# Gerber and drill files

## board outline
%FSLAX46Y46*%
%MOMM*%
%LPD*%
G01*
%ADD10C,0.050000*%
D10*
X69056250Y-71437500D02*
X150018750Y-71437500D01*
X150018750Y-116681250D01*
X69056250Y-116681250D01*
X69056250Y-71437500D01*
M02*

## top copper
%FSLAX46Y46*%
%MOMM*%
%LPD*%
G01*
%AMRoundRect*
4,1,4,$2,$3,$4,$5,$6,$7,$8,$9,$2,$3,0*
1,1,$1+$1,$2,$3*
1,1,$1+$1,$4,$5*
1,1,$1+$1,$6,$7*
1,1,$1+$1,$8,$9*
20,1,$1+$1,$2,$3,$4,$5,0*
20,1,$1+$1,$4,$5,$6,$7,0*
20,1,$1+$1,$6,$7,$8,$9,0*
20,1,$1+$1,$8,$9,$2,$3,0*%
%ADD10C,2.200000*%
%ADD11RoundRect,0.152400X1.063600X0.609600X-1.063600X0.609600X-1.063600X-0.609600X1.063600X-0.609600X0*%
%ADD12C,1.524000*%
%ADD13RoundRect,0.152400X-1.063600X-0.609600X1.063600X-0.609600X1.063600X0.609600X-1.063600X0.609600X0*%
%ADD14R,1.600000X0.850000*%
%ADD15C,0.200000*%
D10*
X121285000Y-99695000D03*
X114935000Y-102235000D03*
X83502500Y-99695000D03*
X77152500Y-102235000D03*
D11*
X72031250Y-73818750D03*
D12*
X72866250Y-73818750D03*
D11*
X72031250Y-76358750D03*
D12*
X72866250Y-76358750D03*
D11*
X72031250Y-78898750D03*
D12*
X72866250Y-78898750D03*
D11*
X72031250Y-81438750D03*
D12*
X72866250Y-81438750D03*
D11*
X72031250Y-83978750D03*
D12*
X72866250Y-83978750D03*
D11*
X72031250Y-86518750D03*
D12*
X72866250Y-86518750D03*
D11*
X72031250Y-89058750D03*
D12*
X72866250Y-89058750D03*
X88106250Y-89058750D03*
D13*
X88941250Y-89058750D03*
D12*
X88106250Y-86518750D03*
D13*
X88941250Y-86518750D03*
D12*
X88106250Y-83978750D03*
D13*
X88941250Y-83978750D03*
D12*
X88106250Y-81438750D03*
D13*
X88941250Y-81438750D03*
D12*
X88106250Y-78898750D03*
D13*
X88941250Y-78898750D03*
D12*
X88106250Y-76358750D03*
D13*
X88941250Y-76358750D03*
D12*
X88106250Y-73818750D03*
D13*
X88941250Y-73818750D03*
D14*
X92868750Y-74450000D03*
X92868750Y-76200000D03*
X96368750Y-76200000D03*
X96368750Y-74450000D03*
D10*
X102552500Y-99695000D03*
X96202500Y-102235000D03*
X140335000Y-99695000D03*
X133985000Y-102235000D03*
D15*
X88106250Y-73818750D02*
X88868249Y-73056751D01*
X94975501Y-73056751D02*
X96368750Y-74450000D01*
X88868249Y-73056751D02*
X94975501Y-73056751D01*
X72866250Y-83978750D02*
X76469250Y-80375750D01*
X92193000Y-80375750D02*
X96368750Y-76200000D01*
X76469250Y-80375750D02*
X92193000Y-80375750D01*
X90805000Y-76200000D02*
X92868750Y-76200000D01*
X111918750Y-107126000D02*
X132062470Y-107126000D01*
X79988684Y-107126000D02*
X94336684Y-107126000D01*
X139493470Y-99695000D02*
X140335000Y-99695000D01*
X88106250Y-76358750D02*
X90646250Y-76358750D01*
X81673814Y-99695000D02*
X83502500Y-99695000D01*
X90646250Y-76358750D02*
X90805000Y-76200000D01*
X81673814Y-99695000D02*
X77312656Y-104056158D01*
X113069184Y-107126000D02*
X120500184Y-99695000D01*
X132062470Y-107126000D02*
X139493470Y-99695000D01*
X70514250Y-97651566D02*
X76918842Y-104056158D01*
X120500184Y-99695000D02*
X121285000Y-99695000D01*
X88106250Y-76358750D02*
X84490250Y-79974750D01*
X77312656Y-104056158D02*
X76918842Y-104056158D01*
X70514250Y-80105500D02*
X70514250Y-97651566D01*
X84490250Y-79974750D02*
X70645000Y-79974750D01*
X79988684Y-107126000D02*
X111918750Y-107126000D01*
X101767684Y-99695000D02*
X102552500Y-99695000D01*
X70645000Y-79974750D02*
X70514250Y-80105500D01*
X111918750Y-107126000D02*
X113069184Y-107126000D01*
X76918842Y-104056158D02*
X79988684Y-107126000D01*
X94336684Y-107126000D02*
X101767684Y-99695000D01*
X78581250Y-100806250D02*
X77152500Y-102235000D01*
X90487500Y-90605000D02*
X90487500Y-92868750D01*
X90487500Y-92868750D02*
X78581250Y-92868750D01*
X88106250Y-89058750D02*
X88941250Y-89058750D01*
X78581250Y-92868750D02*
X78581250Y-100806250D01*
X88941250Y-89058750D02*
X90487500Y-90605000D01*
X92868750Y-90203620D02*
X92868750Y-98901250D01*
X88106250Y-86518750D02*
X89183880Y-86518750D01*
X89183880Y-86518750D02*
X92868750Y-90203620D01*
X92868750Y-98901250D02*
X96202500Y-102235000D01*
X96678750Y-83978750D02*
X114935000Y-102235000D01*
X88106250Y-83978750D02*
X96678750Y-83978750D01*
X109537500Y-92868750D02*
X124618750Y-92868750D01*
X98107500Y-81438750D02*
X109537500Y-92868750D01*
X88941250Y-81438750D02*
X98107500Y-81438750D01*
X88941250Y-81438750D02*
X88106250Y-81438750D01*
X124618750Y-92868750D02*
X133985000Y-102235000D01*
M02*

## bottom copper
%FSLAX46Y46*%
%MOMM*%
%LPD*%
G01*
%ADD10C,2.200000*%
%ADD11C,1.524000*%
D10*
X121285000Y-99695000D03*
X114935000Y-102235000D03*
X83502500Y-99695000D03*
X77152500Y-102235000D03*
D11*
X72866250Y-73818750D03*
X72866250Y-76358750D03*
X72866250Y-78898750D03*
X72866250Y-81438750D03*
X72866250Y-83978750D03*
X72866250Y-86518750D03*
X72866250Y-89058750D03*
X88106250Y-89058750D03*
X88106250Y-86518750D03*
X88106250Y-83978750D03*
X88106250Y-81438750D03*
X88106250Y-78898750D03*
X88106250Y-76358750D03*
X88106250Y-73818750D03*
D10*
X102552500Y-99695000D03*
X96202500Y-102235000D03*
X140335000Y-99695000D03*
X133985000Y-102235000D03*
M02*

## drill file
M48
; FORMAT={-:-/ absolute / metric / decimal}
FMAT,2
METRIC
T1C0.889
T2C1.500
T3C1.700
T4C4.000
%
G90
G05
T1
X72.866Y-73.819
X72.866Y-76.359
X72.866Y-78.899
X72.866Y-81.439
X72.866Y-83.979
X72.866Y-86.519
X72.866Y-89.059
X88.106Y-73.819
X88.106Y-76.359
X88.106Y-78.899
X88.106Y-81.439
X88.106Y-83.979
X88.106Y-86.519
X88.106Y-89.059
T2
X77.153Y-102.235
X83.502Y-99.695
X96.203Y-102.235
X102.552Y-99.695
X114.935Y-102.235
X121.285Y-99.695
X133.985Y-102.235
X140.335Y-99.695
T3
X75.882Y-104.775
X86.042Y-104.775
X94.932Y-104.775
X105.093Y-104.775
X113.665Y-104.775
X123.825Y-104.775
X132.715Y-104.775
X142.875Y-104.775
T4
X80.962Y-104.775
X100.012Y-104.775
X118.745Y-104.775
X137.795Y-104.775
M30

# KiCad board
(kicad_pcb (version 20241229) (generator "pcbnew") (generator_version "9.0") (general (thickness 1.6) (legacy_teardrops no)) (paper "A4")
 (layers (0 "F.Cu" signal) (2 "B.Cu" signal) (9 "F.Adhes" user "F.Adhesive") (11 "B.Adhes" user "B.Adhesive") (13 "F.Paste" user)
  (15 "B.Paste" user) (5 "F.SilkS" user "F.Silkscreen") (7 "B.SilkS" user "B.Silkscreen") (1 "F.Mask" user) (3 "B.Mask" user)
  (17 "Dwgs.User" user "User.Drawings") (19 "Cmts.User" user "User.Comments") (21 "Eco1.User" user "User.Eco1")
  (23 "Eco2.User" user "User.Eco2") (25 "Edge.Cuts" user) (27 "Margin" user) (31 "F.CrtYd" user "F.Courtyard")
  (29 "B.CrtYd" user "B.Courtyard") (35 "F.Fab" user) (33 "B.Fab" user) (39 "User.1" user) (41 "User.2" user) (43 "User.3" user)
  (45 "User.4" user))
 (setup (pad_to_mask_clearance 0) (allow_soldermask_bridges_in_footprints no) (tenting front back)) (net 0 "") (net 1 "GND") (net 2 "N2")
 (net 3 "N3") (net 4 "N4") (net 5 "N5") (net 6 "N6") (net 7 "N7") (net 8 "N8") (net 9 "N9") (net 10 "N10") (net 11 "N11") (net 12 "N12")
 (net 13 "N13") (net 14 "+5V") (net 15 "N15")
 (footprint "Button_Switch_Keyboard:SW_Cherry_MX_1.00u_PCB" (layer "F.Cu") (at 121.285 99.695)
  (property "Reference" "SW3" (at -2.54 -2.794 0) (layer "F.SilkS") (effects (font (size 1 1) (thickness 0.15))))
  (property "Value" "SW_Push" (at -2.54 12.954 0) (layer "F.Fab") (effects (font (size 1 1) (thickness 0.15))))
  (pad "" np_thru_hole circle (at -7.62 5.08) (size 1.7 1.7) (drill 1.7) (layers "*.Cu" "*.Mask"))
  (pad "" np_thru_hole circle (at -2.54 5.08) (size 4 4) (drill 4) (layers "*.Cu" "*.Mask"))
  (pad "" np_thru_hole circle (at 2.54 5.08) (size 1.7 1.7) (drill 1.7) (layers "*.Cu" "*.Mask"))
  (pad "1" thru_hole circle (at 0 0) (size 2.2 2.2) (drill 1.5) (layers "*.Cu" "*.Mask") (remove_unused_layers no) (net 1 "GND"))
  (pad "2" thru_hole circle (at -6.35 2.54) (size 2.2 2.2) (drill 1.5) (layers "*.Cu" "*.Mask") (remove_unused_layers no) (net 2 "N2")))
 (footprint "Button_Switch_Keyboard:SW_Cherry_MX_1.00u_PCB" (layer "F.Cu") (at 83.5025 99.695)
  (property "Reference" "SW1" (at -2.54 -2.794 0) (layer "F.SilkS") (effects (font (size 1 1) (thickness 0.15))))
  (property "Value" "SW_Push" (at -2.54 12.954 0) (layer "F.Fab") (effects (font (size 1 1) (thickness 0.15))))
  (pad "" np_thru_hole circle (at -7.62 5.08) (size 1.7 1.7) (drill 1.7) (layers "*.Cu" "*.Mask"))
  (pad "" np_thru_hole circle (at -2.54 5.08) (size 4 4) (drill 4) (layers "*.Cu" "*.Mask"))
  (pad "" np_thru_hole circle (at 2.54 5.08) (size 1.7 1.7) (drill 1.7) (layers "*.Cu" "*.Mask"))
  (pad "1" thru_hole circle (at 0 0) (size 2.2 2.2) (drill 1.5) (layers "*.Cu" "*.Mask") (remove_unused_layers no) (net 1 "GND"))
  (pad "2" thru_hole circle (at -6.35 2.54) (size 2.2 2.2) (drill 1.5) (layers "*.Cu" "*.Mask") (remove_unused_layers no) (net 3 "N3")))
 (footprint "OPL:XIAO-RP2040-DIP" (layer "F.Cu") (at 80.48625 81.43875)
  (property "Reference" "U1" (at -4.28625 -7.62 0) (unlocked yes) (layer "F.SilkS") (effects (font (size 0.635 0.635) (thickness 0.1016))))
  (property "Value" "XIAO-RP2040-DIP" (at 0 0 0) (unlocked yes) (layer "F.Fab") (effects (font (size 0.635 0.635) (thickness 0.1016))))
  (pad "1" smd roundrect (at -8.455 -7.62 180) (size 2.432 1.524) (layers "F.Cu" "F.Mask") (roundrect_rratio 0.1) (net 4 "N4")
   (thermal_bridge_angle 45))
  (pad "1" thru_hole circle (at -7.62 -7.62 180) (size 1.524 1.524) (drill 0.889) (layers "*.Cu" "*.Mask") (remove_unused_layers no)
   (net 4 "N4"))
  (pad "2" smd roundrect (at -8.455 -5.08 180) (size 2.432 1.524) (layers "F.Cu" "F.Mask") (roundrect_rratio 0.1) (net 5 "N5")
   (thermal_bridge_angle 45))
  (pad "2" thru_hole circle (at -7.62 -5.08 180) (size 1.524 1.524) (drill 0.889) (layers "*.Cu" "*.Mask") (remove_unused_layers no)
   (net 5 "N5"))
  (pad "3" smd roundrect (at -8.455 -2.54 180) (size 2.432 1.524) (layers "F.Cu" "F.Mask") (roundrect_rratio 0.1) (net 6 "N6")
   (thermal_bridge_angle 45))
  (pad "3" thru_hole circle (at -7.62 -2.54 180) (size 1.524 1.524) (drill 0.889) (layers "*.Cu" "*.Mask") (remove_unused_layers no)
   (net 6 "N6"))
  (pad "4" smd roundrect (at -8.455 0 180) (size 2.432 1.524) (layers "F.Cu" "F.Mask") (roundrect_rratio 0.1) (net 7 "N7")
   (thermal_bridge_angle 45))
  (pad "4" thru_hole circle (at -7.62 0 180) (size 1.524 1.524) (drill 0.889) (layers "*.Cu" "*.Mask") (remove_unused_layers no)
   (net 7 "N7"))
  (pad "5" smd roundrect (at -8.455 2.54 180) (size 2.432 1.524) (layers "F.Cu" "F.Mask") (roundrect_rratio 0.1) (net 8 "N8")
   (thermal_bridge_angle 45))
  (pad "5" thru_hole circle (at -7.62 2.54 180) (size 1.524 1.524) (drill 0.889) (layers "*.Cu" "*.Mask") (remove_unused_layers no)
   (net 8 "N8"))
  (pad "6" smd roundrect (at -8.455 5.08 180) (size 2.432 1.524) (layers "F.Cu" "F.Mask") (roundrect_rratio 0.1) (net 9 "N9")
   (thermal_bridge_angle 45))
  (pad "6" thru_hole circle (at -7.62 5.08 180) (size 1.524 1.524) (drill 0.889) (layers "*.Cu" "*.Mask") (remove_unused_layers no)
   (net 9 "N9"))
  (pad "7" smd roundrect (at -8.455 7.62 180) (size 2.432 1.524) (layers "F.Cu" "F.Mask") (roundrect_rratio 0.1) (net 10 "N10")
   (thermal_bridge_angle 45))
  (pad "7" thru_hole circle (at -7.62 7.62 180) (size 1.524 1.524) (drill 0.889) (layers "*.Cu" "*.Mask") (remove_unused_layers no)
   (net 10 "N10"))
  (pad "8" thru_hole circle (at 7.62 7.62) (size 1.524 1.524) (drill 0.889) (layers "*.Cu" "*.Mask") (remove_unused_layers no) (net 3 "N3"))
  (pad "8" smd roundrect (at 8.455 7.62) (size 2.432 1.524) (layers "F.Cu" "F.Mask") (roundrect_rratio 0.1) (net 3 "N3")
   (thermal_bridge_angle 45))
  (pad "9" thru_hole circle (at 7.62 5.08) (size 1.524 1.524) (drill 0.889) (layers "*.Cu" "*.Mask") (remove_unused_layers no)
   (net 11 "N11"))
  (pad "9" smd roundrect (at 8.455 5.08) (size 2.432 1.524) (layers "F.Cu" "F.Mask") (roundrect_rratio 0.1) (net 11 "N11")
   (thermal_bridge_angle 45))
  (pad "10" thru_hole circle (at 7.62 2.54) (size 1.524 1.524) (drill 0.889) (layers "*.Cu" "*.Mask") (remove_unused_layers no) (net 2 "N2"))
  (pad "10" smd roundrect (at 8.455 2.54) (size 2.432 1.524) (layers "F.Cu" "F.Mask") (roundrect_rratio 0.1) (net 2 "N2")
   (thermal_bridge_angle 45))
  (pad "11" thru_hole circle (at 7.62 0) (size 1.524 1.524) (drill 0.889) (layers "*.Cu" "*.Mask") (remove_unused_layers no) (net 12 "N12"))
  (pad "11" smd roundrect (at 8.455 0) (size 2.432 1.524) (layers "F.Cu" "F.Mask") (roundrect_rratio 0.1) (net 12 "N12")
   (thermal_bridge_angle 45))
  (pad "12" thru_hole circle (at 7.62 -2.54) (size 1.524 1.524) (drill 0.889) (layers "*.Cu" "*.Mask") (remove_unused_layers no)
   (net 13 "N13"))
  (pad "12" smd roundrect (at 8.455 -2.54) (size 2.432 1.524) (layers "F.Cu" "F.Mask") (roundrect_rratio 0.1) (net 13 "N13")
   (thermal_bridge_angle 45))
  (pad "13" thru_hole circle (at 7.62 -5.08) (size 1.524 1.524) (drill 0.889) (layers "*.Cu" "*.Mask") (remove_unused_layers no)
   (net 1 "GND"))
  (pad "13" smd roundrect (at 8.455 -5.08) (size 2.432 1.524) (layers "F.Cu" "F.Mask") (roundrect_rratio 0.1) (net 1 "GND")
   (thermal_bridge_angle 45))
  (pad "14" thru_hole circle (at 7.62 -7.62) (size 1.524 1.524) (drill 0.889) (layers "*.Cu" "*.Mask") (remove_unused_layers no)
   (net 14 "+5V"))
  (pad "14" smd roundrect (at 8.455 -7.62) (size 2.432 1.524) (layers "F.Cu" "F.Mask") (roundrect_rratio 0.1) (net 14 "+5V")
   (thermal_bridge_angle 45)))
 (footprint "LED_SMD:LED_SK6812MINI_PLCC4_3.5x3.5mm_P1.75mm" (layer "F.Cu") (at 94.61875 75.325)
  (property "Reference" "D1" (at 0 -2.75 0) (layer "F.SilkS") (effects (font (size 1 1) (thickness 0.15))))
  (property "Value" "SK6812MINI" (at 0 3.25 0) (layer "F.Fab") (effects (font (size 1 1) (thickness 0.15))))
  (pad "1" smd rect (at -1.75 -0.875) (size 1.6 0.85) (layers "F.Cu" "F.Mask" "F.Paste") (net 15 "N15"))
  (pad "2" smd rect (at -1.75 0.875) (size 1.6 0.85) (layers "F.Cu" "F.Mask" "F.Paste") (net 1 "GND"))
  (pad "3" smd rect (at 1.75 0.875) (size 1.6 0.85) (layers "F.Cu" "F.Mask" "F.Paste") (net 8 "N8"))
  (pad "4" smd rect (at 1.75 -0.875) (size 1.6 0.85) (layers "F.Cu" "F.Mask" "F.Paste") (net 14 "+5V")))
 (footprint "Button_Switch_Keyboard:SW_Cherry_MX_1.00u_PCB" (layer "F.Cu") (at 102.5525 99.695)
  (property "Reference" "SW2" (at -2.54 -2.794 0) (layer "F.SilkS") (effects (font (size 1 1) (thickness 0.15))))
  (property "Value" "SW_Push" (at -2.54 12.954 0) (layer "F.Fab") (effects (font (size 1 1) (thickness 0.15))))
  (pad "" np_thru_hole circle (at -7.62 5.08) (size 1.7 1.7) (drill 1.7) (layers "*.Cu" "*.Mask"))
  (pad "" np_thru_hole circle (at -2.54 5.08) (size 4 4) (drill 4) (layers "*.Cu" "*.Mask"))
  (pad "" np_thru_hole circle (at 2.54 5.08) (size 1.7 1.7) (drill 1.7) (layers "*.Cu" "*.Mask"))
  (pad "1" thru_hole circle (at 0 0) (size 2.2 2.2) (drill 1.5) (layers "*.Cu" "*.Mask") (remove_unused_layers no) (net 1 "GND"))
  (pad "2" thru_hole circle (at -6.35 2.54) (size 2.2 2.2) (drill 1.5) (layers "*.Cu" "*.Mask") (remove_unused_layers no) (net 11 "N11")))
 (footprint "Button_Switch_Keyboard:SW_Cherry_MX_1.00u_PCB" (layer "F.Cu") (at 140.335 99.695)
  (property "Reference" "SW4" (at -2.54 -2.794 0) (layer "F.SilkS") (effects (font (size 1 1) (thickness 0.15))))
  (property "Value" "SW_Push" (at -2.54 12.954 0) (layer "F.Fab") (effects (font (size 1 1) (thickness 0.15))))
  (pad "" np_thru_hole circle (at -7.62 5.08) (size 1.7 1.7) (drill 1.7) (layers "*.Cu" "*.Mask"))
  (pad "" np_thru_hole circle (at -2.54 5.08) (size 4 4) (drill 4) (layers "*.Cu" "*.Mask"))
  (pad "" np_thru_hole circle (at 2.54 5.08) (size 1.7 1.7) (drill 1.7) (layers "*.Cu" "*.Mask"))
  (pad "1" thru_hole circle (at 0 0) (size 2.2 2.2) (drill 1.5) (layers "*.Cu" "*.Mask") (remove_unused_layers no) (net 1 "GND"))
  (pad "2" thru_hole circle (at -6.35 2.54) (size 2.2 2.2) (drill 1.5) (layers "*.Cu" "*.Mask") (remove_unused_layers no) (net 12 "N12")))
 (gr_rect (start 69.05625 71.4375) (end 150.01875 116.68125) (stroke (width 0.05) (type default)) (fill no) (layer "Edge.Cuts"))
 (segment (start 88.10625 73.81875) (end 88.868249 73.056751) (width 0.2) (layer "F.Cu") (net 14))
 (segment (start 94.975501 73.056751) (end 96.36875 74.45) (width 0.2) (layer "F.Cu") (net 14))
 (segment (start 88.868249 73.056751) (end 94.975501 73.056751) (width 0.2) (layer "F.Cu") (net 14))
 (segment (start 72.86625 83.97875) (end 76.46925 80.37575) (width 0.2) (layer "F.Cu") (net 8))
 (segment (start 92.193 80.37575) (end 96.36875 76.2) (width 0.2) (layer "F.Cu") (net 8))
 (segment (start 76.46925 80.37575) (end 92.193 80.37575) (width 0.2) (layer "F.Cu") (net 8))
 (segment (start 90.805 76.2) (end 92.86875 76.2) (width 0.2) (layer "F.Cu") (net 1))
 (segment (start 111.91875 107.126) (end 132.06247 107.126) (width 0.2) (layer "F.Cu") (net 1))
 (segment (start 79.988684 107.126) (end 94.336684 107.126) (width 0.2) (layer "F.Cu") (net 1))
 (segment (start 139.49347 99.695) (end 140.335 99.695) (width 0.2) (layer "F.Cu") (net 1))
 (segment (start 88.10625 76.35875) (end 90.64625 76.35875) (width 0.2) (layer "F.Cu") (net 1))
 (segment (start 81.673814 99.695) (end 83.5025 99.695) (width 0.2) (layer "F.Cu") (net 1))
 (segment (start 90.64625 76.35875) (end 90.805 76.2) (width 0.2) (layer "F.Cu") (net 1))
 (segment (start 81.673814 99.695) (end 77.312656 104.056158) (width 0.2) (layer "F.Cu") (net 1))
 (segment (start 113.069184 107.126) (end 120.500184 99.695) (width 0.2) (layer "F.Cu") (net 1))
 (segment (start 132.06247 107.126) (end 139.49347 99.695) (width 0.2) (layer "F.Cu") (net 1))
 (segment (start 70.51425 97.651566) (end 76.918842 104.056158) (width 0.2) (layer "F.Cu") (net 1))
 (segment (start 120.500184 99.695) (end 121.285 99.695) (width 0.2) (layer "F.Cu") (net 1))
 (segment (start 88.10625 76.35875) (end 84.49025 79.97475) (width 0.2) (layer "F.Cu") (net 1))
 (segment (start 77.312656 104.056158) (end 76.918842 104.056158) (width 0.2) (layer "F.Cu") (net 1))
 (segment (start 70.51425 80.1055) (end 70.51425 97.651566) (width 0.2) (layer "F.Cu") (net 1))
 (segment (start 84.49025 79.97475) (end 70.645 79.97475) (width 0.2) (layer "F.Cu") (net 1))
 (segment (start 79.988684 107.126) (end 111.91875 107.126) (width 0.2) (layer "F.Cu") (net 1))
 (segment (start 101.767684 99.695) (end 102.5525 99.695) (width 0.2) (layer "F.Cu") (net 1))
 (segment (start 70.645 79.97475) (end 70.51425 80.1055) (width 0.2) (layer "F.Cu") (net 1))
 (segment (start 111.91875 107.126) (end 113.069184 107.126) (width 0.2) (layer "F.Cu") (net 1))
 (segment (start 76.918842 104.056158) (end 79.988684 107.126) (width 0.2) (layer "F.Cu") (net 1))
 (segment (start 94.336684 107.126) (end 101.767684 99.695) (width 0.2) (layer "F.Cu") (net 1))
 (segment (start 78.58125 100.80625) (end 77.1525 102.235) (width 0.2) (layer "F.Cu") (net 3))
 (segment (start 90.4875 90.605) (end 90.4875 92.86875) (width 0.2) (layer "F.Cu") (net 3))
 (segment (start 90.4875 92.86875) (end 78.58125 92.86875) (width 0.2) (layer "F.Cu") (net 3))
 (segment (start 88.10625 89.05875) (end 88.94125 89.05875) (width 0.2) (layer "F.Cu") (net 3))
 (segment (start 78.58125 92.86875) (end 78.58125 100.80625) (width 0.2) (layer "F.Cu") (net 3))
 (segment (start 88.94125 89.05875) (end 90.4875 90.605) (width 0.2) (layer "F.Cu") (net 3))
 (segment (start 92.86875 90.20362) (end 92.86875 98.90125) (width 0.2) (layer "F.Cu") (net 11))
 (segment (start 88.10625 86.51875) (end 89.18388 86.51875) (width 0.2) (layer "F.Cu") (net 11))
 (segment (start 89.18388 86.51875) (end 92.86875 90.20362) (width 0.2) (layer "F.Cu") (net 11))
 (segment (start 92.86875 98.90125) (end 96.2025 102.235) (width 0.2) (layer "F.Cu") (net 11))
 (segment (start 96.67875 83.97875) (end 114.935 102.235) (width 0.2) (layer "F.Cu") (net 2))
 (segment (start 88.10625 83.97875) (end 96.67875 83.97875) (width 0.2) (layer "F.Cu") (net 2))
 (segment (start 109.5375 92.86875) (end 124.61875 92.86875) (width 0.2) (layer "F.Cu") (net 12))
 (segment (start 98.1075 81.43875) (end 109.5375 92.86875) (width 0.2) (layer "F.Cu") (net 12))
 (segment (start 88.94125 81.43875) (end 98.1075 81.43875) (width 0.2) (layer "F.Cu") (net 12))
 (segment (start 88.94125 81.43875) (end 88.10625 81.43875) (width 0.2) (layer "F.Cu") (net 12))
 (segment (start 124.61875 92.86875) (end 133.985 102.235) (width 0.2) (layer "F.Cu") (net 12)))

